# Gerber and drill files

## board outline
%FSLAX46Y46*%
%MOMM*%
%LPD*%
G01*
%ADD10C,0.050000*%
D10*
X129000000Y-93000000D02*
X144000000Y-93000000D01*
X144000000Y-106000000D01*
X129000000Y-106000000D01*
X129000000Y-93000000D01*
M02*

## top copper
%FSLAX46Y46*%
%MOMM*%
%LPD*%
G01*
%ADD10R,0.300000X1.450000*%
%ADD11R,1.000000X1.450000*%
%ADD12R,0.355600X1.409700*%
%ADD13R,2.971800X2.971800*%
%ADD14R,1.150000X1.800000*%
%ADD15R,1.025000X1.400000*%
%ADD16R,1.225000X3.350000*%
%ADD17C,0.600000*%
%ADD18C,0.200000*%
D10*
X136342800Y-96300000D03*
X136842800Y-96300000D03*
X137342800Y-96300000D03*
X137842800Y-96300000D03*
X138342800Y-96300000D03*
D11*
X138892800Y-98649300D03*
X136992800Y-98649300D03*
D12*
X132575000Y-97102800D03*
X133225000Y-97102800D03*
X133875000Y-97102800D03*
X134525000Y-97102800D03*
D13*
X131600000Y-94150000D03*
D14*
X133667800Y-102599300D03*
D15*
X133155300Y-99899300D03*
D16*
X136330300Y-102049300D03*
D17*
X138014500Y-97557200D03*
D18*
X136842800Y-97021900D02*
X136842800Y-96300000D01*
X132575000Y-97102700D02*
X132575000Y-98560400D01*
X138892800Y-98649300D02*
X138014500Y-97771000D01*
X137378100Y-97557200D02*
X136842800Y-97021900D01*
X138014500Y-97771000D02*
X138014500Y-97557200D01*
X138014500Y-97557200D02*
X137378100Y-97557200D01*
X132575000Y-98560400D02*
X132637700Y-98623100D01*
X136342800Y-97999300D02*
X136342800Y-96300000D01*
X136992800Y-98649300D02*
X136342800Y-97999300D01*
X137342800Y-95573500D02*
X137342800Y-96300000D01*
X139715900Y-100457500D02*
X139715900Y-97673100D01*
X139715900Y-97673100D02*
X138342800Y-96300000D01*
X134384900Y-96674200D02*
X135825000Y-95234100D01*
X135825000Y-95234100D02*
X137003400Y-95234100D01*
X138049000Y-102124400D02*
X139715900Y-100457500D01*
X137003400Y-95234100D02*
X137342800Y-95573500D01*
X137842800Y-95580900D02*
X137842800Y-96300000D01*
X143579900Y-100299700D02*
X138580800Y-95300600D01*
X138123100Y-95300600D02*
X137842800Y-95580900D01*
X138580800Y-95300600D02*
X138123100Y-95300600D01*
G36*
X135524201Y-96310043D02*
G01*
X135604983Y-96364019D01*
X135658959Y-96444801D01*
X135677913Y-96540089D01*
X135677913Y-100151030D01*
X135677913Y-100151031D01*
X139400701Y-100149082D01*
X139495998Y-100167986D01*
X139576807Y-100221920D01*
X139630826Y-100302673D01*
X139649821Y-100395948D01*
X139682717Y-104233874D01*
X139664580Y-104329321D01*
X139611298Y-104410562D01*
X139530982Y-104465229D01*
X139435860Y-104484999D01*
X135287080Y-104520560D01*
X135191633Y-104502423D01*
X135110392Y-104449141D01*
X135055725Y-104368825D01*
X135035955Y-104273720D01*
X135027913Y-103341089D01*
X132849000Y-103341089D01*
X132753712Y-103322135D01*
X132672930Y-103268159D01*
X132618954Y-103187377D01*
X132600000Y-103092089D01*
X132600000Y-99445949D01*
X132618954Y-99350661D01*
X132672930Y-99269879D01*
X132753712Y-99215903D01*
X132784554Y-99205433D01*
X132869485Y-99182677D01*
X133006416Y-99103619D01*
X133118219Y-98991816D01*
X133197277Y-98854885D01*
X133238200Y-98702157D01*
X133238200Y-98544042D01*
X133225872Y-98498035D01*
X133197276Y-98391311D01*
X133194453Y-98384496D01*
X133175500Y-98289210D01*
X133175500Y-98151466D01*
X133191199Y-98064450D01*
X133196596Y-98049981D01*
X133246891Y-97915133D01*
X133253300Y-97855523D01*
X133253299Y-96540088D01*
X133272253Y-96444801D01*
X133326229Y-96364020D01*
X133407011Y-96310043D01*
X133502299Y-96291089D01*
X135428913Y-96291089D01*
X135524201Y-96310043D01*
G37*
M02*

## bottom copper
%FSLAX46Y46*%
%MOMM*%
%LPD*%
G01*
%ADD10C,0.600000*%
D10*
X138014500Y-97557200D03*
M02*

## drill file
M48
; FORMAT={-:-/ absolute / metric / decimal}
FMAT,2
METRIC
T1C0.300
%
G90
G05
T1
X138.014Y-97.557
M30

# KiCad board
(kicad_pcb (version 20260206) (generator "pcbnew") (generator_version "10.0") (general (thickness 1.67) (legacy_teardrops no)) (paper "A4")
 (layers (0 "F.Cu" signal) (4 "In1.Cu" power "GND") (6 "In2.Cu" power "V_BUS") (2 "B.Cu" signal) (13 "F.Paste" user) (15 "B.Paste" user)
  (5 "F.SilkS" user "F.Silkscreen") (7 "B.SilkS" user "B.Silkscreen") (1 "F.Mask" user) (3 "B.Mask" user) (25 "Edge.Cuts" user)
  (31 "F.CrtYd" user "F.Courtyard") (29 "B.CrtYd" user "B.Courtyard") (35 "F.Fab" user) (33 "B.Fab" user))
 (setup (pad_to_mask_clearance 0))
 (gr_rect (start 129 93) (end 144 106) (stroke (width 0.05) (type default)) (fill no) (layer "Edge.Cuts"))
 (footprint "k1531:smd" (layer "F.Cu") (at 136.3428 96.3) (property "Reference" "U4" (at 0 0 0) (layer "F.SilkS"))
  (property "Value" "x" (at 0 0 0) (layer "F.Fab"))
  (pad "1" smd rect (at 0 0) (size 0.3 1.45) (layers "F.Cu" "F.Mask") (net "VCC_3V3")))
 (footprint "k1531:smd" (layer "F.Cu") (at 136.8428 96.3) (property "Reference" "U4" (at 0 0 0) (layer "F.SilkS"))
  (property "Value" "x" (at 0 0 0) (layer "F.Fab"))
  (pad "1" smd rect (at 0 0) (size 0.3 1.45) (layers "F.Cu" "F.Mask") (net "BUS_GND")))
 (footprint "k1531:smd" (layer "F.Cu") (at 137.3428 96.3) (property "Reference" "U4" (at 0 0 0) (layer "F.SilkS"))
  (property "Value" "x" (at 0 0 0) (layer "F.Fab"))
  (pad "1" smd rect (at 0 0) (size 0.3 1.45) (layers "F.Cu" "F.Mask") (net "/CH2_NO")))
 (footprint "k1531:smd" (layer "F.Cu") (at 137.8428 96.3) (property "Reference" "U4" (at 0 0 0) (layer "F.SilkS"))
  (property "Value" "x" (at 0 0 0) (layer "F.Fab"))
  (pad "1" smd rect (at 0 0) (size 0.3 1.45) (layers "F.Cu" "F.Mask") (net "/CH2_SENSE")))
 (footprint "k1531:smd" (layer "F.Cu") (at 138.3428 96.3) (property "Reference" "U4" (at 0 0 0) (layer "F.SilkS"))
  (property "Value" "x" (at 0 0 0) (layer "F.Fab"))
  (pad "1" smd rect (at 0 0) (size 0.3 1.45) (layers "F.Cu" "F.Mask") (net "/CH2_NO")))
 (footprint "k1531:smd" (layer "F.Cu") (at 138.8928 98.6493) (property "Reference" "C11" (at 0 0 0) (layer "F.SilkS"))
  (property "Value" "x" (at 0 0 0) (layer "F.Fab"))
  (pad "1" smd rect (at 0 0) (size 1.0 1.45) (layers "F.Cu" "F.Mask") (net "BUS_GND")))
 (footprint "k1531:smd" (layer "F.Cu") (at 136.9928 98.6493) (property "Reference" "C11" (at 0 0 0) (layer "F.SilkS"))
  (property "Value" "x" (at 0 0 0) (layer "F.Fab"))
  (pad "1" smd rect (at 0 0) (size 1.0 1.45) (layers "F.Cu" "F.Mask") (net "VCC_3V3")))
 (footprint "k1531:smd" (layer "F.Cu") (at 132.575 97.1028) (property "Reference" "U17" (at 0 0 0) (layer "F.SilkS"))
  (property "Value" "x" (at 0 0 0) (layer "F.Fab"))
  (pad "1" smd rect (at 0 0) (size 0.3556 1.4097) (layers "F.Cu" "F.Mask") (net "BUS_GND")))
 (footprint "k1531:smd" (layer "F.Cu") (at 133.225 97.1028) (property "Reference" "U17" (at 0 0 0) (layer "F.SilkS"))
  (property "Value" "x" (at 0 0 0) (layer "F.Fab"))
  (pad "1" smd rect (at 0 0) (size 0.3556 1.4097) (layers "F.Cu" "F.Mask") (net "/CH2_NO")))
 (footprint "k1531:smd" (layer "F.Cu") (at 133.875 97.1028) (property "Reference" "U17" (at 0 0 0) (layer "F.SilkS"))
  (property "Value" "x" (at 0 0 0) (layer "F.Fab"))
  (pad "1" smd rect (at 0 0) (size 0.3556 1.4097) (layers "F.Cu" "F.Mask") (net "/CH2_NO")))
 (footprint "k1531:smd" (layer "F.Cu") (at 134.525 97.1028) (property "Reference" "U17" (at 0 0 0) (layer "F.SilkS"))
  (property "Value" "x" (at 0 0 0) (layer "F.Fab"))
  (pad "1" smd rect (at 0 0) (size 0.3556 1.4097) (layers "F.Cu" "F.Mask") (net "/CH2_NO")))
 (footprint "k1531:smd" (layer "F.Cu") (at 131.6 94.15) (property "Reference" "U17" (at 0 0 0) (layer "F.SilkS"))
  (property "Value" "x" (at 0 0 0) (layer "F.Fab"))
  (pad "1" smd rect (at 0 0) (size 2.9718 2.9718) (layers "F.Cu" "F.Mask") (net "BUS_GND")))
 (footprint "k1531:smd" (layer "F.Cu") (at 133.6678 102.5993) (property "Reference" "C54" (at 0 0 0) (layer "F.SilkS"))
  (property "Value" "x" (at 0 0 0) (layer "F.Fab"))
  (pad "1" smd rect (at 0 0) (size 1.15 1.8) (layers "F.Cu" "F.Mask") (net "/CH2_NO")))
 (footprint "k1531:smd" (layer "F.Cu") (at 133.1553 99.8993) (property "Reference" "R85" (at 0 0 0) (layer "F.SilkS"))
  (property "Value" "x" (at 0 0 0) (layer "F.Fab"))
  (pad "1" smd rect (at 0 0) (size 1.025 1.4) (layers "F.Cu" "F.Mask") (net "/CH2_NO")))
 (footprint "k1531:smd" (layer "F.Cu") (at 136.3303 102.0493) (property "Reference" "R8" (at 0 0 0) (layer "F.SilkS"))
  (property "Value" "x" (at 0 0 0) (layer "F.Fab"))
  (pad "1" smd rect (at 0 0) (size 1.225 3.35) (layers "F.Cu" "F.Mask") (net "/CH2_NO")))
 (segment (start 136.8428 97.0219) (end 136.8428 96.3) (width 0.2) (layer "F.Cu") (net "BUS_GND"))
 (segment (start 132.575 97.1027) (end 132.575 98.5604) (width 0.2) (layer "F.Cu") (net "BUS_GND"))
 (segment (start 138.8928 98.6493) (end 138.0145 97.771) (width 0.2) (layer "F.Cu") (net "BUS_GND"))
 (segment (start 137.3781 97.5572) (end 136.8428 97.0219) (width 0.2) (layer "F.Cu") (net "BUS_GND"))
 (segment (start 138.0145 97.771) (end 138.0145 97.5572) (width 0.2) (layer "F.Cu") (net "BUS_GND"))
 (segment (start 138.0145 97.5572) (end 137.3781 97.5572) (width 0.2) (layer "F.Cu") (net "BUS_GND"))
 (segment (start 132.575 98.5604) (end 132.6377 98.6231) (width 0.2) (layer "F.Cu") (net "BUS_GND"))
 (segment (start 136.3428 97.9993) (end 136.3428 96.3) (width 0.2) (layer "F.Cu") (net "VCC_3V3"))
 (segment (start 136.9928 98.6493) (end 136.3428 97.9993) (width 0.2) (layer "F.Cu") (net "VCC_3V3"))
 (segment (start 137.3428 95.5735) (end 137.3428 96.3) (width 0.2) (layer "F.Cu") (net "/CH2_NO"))
 (segment (start 139.7159 100.4575) (end 139.7159 97.6731) (width 0.2) (layer "F.Cu") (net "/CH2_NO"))
 (segment (start 139.7159 97.6731) (end 138.3428 96.3) (width 0.2) (layer "F.Cu") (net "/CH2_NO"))
 (segment (start 134.3849 96.6742) (end 135.825 95.2341) (width 0.2) (layer "F.Cu") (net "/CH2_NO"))
 (segment (start 135.825 95.2341) (end 137.0034 95.2341) (width 0.2) (layer "F.Cu") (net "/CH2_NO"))
 (segment (start 138.049 102.1244) (end 139.7159 100.4575) (width 0.2) (layer "F.Cu") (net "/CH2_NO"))
 (segment (start 137.0034 95.2341) (end 137.3428 95.5735) (width 0.2) (layer "F.Cu") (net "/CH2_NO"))
 (segment (start 137.8428 95.5809) (end 137.8428 96.3) (width 0.2) (layer "F.Cu") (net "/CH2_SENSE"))
 (segment (start 143.5799 100.2997) (end 138.5808 95.3006) (width 0.2) (layer "F.Cu") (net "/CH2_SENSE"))
 (segment (start 138.1231 95.3006) (end 137.8428 95.5809) (width 0.2) (layer "F.Cu") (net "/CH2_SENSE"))
 (segment (start 138.5808 95.3006) (end 138.1231 95.3006) (width 0.2) (layer "F.Cu") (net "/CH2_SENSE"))
 (via (at 138.0145 97.5572) (size 0.6) (drill 0.3) (layers "F.Cu" "B.Cu") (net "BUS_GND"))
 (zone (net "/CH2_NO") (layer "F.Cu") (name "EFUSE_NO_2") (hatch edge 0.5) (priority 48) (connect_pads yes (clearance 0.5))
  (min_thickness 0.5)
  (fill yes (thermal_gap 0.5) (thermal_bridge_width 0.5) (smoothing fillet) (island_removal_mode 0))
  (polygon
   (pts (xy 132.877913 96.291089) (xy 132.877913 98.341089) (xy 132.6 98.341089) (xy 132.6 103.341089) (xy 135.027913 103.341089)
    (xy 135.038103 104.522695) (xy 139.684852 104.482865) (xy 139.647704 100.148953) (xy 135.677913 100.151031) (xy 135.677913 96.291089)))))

